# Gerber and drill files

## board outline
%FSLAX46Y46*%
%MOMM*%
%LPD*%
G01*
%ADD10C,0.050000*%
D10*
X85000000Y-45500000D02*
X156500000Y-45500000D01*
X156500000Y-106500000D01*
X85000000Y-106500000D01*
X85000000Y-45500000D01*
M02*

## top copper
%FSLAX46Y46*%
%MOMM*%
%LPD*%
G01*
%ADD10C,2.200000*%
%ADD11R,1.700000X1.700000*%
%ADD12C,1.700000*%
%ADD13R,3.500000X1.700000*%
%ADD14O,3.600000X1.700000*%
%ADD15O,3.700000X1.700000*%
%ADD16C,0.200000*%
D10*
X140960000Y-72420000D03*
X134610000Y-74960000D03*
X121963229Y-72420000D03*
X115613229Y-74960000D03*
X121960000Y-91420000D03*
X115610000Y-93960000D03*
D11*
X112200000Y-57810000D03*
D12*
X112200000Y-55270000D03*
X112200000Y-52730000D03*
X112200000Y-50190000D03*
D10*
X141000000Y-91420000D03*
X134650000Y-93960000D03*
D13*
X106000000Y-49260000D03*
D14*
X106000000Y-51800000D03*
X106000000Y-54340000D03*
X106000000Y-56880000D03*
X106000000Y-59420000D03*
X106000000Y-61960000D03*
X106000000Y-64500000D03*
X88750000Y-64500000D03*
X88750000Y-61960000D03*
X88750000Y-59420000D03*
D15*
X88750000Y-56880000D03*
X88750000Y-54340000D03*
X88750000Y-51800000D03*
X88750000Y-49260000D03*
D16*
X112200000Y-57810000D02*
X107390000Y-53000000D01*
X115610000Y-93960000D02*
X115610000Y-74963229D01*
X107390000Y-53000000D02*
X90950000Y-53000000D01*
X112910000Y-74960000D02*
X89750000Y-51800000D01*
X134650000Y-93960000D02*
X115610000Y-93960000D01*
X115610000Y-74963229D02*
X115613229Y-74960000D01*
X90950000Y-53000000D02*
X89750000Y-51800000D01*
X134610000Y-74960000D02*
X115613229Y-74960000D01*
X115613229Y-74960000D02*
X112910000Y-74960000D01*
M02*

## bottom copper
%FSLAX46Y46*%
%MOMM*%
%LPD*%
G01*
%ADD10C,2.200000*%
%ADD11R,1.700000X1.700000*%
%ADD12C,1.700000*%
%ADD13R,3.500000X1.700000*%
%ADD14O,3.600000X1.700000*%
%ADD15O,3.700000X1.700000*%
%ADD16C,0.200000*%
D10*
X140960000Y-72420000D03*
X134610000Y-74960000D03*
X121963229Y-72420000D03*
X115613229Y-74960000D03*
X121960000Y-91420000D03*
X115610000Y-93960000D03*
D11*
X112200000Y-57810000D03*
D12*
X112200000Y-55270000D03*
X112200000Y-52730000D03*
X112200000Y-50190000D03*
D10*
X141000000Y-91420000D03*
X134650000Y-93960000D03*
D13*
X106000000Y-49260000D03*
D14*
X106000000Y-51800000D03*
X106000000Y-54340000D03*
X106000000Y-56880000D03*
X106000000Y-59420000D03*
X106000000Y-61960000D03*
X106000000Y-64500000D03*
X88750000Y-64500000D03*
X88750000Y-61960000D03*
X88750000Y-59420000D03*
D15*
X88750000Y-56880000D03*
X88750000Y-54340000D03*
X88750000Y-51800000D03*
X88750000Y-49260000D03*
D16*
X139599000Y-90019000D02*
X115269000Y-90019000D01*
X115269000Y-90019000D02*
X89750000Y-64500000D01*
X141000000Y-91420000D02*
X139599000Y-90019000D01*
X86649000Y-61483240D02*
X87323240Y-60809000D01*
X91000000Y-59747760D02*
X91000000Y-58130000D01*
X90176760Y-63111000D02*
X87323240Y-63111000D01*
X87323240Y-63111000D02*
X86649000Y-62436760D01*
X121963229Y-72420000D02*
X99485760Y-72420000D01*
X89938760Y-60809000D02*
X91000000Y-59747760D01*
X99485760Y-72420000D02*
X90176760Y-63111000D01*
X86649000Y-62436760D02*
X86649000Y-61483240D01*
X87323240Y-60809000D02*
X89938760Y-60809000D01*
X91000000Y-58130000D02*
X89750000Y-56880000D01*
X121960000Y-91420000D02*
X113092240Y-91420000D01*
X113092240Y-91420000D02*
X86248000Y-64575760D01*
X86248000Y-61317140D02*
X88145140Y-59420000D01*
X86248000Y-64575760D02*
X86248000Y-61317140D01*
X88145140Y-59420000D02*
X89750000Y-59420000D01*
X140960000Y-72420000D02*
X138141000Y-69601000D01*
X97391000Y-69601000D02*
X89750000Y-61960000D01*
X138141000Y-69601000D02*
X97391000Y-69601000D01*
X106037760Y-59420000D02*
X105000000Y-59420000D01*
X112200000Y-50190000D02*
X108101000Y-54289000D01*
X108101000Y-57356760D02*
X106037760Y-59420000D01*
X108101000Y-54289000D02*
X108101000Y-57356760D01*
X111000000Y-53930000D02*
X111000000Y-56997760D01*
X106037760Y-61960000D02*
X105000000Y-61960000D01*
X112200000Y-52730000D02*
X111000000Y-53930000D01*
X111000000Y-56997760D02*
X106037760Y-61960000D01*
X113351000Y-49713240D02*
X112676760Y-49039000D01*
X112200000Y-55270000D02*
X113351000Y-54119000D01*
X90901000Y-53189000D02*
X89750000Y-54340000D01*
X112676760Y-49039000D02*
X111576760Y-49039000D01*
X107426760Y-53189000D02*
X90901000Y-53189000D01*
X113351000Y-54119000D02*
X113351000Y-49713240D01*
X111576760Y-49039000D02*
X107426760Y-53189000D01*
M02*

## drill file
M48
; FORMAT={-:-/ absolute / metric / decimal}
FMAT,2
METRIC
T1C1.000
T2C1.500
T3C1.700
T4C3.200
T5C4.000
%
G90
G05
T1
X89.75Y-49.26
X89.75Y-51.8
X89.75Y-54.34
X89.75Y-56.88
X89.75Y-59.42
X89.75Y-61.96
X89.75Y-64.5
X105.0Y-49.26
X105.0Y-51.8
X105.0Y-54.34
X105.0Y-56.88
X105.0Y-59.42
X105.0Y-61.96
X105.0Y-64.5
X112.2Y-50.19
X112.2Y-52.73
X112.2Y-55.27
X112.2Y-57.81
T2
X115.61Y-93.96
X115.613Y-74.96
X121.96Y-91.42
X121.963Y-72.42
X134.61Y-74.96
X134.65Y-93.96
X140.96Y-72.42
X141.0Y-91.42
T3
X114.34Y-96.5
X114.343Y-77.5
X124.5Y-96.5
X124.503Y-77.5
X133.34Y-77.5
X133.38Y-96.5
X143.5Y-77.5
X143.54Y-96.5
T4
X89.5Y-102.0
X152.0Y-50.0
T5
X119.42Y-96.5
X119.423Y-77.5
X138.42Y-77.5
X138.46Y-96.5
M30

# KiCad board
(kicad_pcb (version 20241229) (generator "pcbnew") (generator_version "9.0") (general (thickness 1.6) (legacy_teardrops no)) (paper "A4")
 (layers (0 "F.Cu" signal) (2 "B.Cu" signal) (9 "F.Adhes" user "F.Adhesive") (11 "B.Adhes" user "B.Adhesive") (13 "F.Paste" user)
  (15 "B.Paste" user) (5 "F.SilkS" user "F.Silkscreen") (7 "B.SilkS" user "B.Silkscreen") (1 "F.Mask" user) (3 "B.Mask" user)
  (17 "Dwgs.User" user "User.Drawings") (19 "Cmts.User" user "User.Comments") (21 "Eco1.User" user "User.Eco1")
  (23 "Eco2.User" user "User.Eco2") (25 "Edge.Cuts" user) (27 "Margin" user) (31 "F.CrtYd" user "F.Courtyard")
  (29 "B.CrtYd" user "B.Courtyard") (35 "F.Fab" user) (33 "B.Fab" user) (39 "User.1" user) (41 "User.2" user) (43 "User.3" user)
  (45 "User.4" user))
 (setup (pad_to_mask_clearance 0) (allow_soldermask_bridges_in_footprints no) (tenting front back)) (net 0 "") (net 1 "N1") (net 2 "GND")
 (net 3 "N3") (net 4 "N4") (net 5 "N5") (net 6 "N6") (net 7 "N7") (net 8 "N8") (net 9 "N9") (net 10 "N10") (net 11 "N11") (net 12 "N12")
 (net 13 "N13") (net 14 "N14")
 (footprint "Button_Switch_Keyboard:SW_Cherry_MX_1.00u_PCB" (layer "F.Cu") (at 140.96 72.42)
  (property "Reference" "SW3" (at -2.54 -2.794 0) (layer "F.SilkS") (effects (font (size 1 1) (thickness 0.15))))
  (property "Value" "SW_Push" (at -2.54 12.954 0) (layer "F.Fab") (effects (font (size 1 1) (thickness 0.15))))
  (pad "" np_thru_hole circle (at -7.62 5.08) (size 1.7 1.7) (drill 1.7) (layers "*.Cu" "*.Mask"))
  (pad "" np_thru_hole circle (at -2.54 5.08) (size 4 4) (drill 4) (layers "*.Cu" "*.Mask"))
  (pad "" np_thru_hole circle (at 2.54 5.08) (size 1.7 1.7) (drill 1.7) (layers "*.Cu" "*.Mask"))
  (pad "1" thru_hole circle (at 0 0) (size 2.2 2.2) (drill 1.5) (layers "*.Cu" "*.Mask") (remove_unused_layers no) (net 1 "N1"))
  (pad "2" thru_hole circle (at -6.35 2.54) (size 2.2 2.2) (drill 1.5) (layers "*.Cu" "*.Mask") (remove_unused_layers no) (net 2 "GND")))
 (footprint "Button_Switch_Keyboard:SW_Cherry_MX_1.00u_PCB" (layer "F.Cu") (at 121.963229 72.42)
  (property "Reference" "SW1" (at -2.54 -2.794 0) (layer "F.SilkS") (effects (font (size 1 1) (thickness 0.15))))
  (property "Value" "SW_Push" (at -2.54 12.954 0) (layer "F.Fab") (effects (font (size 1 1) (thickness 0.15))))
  (pad "" np_thru_hole circle (at -7.62 5.08) (size 1.7 1.7) (drill 1.7) (layers "*.Cu" "*.Mask"))
  (pad "" np_thru_hole circle (at -2.54 5.08) (size 4 4) (drill 4) (layers "*.Cu" "*.Mask"))
  (pad "" np_thru_hole circle (at 2.54 5.08) (size 1.7 1.7) (drill 1.7) (layers "*.Cu" "*.Mask"))
  (pad "1" thru_hole circle (at 0 0) (size 2.2 2.2) (drill 1.5) (layers "*.Cu" "*.Mask") (remove_unused_layers no) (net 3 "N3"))
  (pad "2" thru_hole circle (at -6.35 2.54) (size 2.2 2.2) (drill 1.5) (layers "*.Cu" "*.Mask") (remove_unused_layers no) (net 2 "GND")))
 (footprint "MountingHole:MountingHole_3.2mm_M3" (layer "F.Cu") (at 152 50)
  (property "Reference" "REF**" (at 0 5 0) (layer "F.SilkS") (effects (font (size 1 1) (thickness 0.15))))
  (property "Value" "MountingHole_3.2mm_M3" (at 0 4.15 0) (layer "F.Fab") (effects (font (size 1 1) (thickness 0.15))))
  (pad "" np_thru_hole circle (at 0 0) (size 3.2 3.2) (drill 3.2) (layers "*.Cu" "*.Mask")))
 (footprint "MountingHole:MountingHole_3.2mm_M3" (layer "F.Cu") (at 89.5 102)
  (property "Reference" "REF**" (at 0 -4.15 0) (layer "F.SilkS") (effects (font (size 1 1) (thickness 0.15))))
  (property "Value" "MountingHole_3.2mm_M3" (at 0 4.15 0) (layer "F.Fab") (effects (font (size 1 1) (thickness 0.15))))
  (pad "" np_thru_hole circle (at 0 0) (size 3.2 3.2) (drill 3.2) (layers "*.Cu" "*.Mask")))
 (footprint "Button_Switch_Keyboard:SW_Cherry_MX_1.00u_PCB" (layer "F.Cu") (at 121.96 91.42)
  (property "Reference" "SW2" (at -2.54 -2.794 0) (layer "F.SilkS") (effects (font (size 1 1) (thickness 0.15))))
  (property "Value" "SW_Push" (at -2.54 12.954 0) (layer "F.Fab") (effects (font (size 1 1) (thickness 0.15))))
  (pad "" np_thru_hole circle (at -7.62 5.08) (size 1.7 1.7) (drill 1.7) (layers "*.Cu" "*.Mask"))
  (pad "" np_thru_hole circle (at -2.54 5.08) (size 4 4) (drill 4) (layers "*.Cu" "*.Mask"))
  (pad "" np_thru_hole circle (at 2.54 5.08) (size 1.7 1.7) (drill 1.7) (layers "*.Cu" "*.Mask"))
  (pad "1" thru_hole circle (at 0 0) (size 2.2 2.2) (drill 1.5) (layers "*.Cu" "*.Mask") (remove_unused_layers no) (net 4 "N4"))
  (pad "2" thru_hole circle (at -6.35 2.54) (size 2.2 2.2) (drill 1.5) (layers "*.Cu" "*.Mask") (remove_unused_layers no) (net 2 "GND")))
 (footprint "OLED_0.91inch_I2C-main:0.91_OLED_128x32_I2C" (layer "F.Cu") (at 110.2 57.81)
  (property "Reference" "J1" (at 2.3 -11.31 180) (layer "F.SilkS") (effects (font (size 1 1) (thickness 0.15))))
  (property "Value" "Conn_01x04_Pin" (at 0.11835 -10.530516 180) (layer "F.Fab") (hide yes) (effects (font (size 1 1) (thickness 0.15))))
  (pad "1" thru_hole rect (at 2 0 180) (size 1.7 1.7) (drill 1) (layers "*.Cu" "*.Mask") (remove_unused_layers no) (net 2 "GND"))
  (pad "2" thru_hole circle (at 2 -2.54 180) (size 1.7 1.7) (drill 1) (layers "*.Cu" "*.Mask") (remove_unused_layers no) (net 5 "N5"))
  (pad "3" thru_hole circle (at 2 -5.08 180) (size 1.7 1.7) (drill 1) (layers "*.Cu" "*.Mask") (remove_unused_layers no) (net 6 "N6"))
  (pad "4" thru_hole circle (at 2 -7.62 180) (size 1.7 1.7) (drill 1) (layers "*.Cu" "*.Mask") (remove_unused_layers no) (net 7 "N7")))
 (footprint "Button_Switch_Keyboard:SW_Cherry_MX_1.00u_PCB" (layer "F.Cu") (at 141 91.42)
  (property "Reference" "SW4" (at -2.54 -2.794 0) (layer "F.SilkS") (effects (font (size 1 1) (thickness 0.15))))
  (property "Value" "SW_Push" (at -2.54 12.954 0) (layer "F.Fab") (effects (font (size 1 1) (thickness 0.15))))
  (pad "" np_thru_hole circle (at -7.62 5.08) (size 1.7 1.7) (drill 1.7) (layers "*.Cu" "*.Mask"))
  (pad "" np_thru_hole circle (at -2.54 5.08) (size 4 4) (drill 4) (layers "*.Cu" "*.Mask"))
  (pad "" np_thru_hole circle (at 2.54 5.08) (size 1.7 1.7) (drill 1.7) (layers "*.Cu" "*.Mask"))
  (pad "1" thru_hole circle (at 0 0) (size 2.2 2.2) (drill 1.5) (layers "*.Cu" "*.Mask") (remove_unused_layers no) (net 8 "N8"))
  (pad "2" thru_hole circle (at -6.35 2.54) (size 2.2 2.2) (drill 1.5) (layers "*.Cu" "*.Mask") (remove_unused_layers no) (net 2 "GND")))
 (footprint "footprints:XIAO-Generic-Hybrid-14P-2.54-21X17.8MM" (layer "B.Cu") (at 97.375 56.88 180)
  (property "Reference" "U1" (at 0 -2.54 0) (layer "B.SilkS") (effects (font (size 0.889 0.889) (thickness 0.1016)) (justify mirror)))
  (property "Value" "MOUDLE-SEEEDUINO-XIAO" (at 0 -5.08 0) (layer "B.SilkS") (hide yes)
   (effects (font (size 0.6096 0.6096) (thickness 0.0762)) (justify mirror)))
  (pad "1" thru_hole rect (at -7.625 7.62 180) (size 3.5 1.7) (drill 1 (offset -1 0)) (layers "*.Cu" "*.Mask") (remove_unused_layers no)
   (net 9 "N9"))
  (pad "2" thru_hole oval (at -7.625 5.08 180) (size 3.6 1.7) (drill 1 (offset -1 0)) (layers "*.Cu" "*.Mask") (remove_unused_layers no)
   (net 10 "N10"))
  (pad "3" thru_hole oval (at -7.625 2.54 180) (size 3.6 1.7) (drill 1 (offset -1 0)) (layers "*.Cu" "*.Mask") (remove_unused_layers no)
   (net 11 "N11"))
  (pad "4" thru_hole oval (at -7.625 0 180) (size 3.6 1.7) (drill 1 (offset -1 0)) (layers "*.Cu" "*.Mask") (remove_unused_layers no)
   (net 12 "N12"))
  (pad "5" thru_hole oval (at -7.625 -2.54 180) (size 3.6 1.7) (drill 1 (offset -1 0)) (layers "*.Cu" "*.Mask") (remove_unused_layers no)
   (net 7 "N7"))
  (pad "6" thru_hole oval (at -7.625 -5.08) (size 3.6 1.7) (drill 1 (offset 1 0)) (layers "*.Cu" "*.Mask") (remove_unused_layers no)
   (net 6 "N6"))
  (pad "7" thru_hole oval (at -7.625 -7.62 180) (size 3.6 1.7) (drill 1 (offset -1 0)) (layers "*.Cu" "*.Mask") (remove_unused_layers no)
   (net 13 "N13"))
  (pad "8" thru_hole oval (at 7.625 -7.62 180) (size 3.6 1.7) (drill 1 (offset 1 0)) (layers "*.Cu" "*.Mask") (remove_unused_layers no)
   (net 8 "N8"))
  (pad "9" thru_hole oval (at 7.625 -5.08 180) (size 3.6 1.7) (drill 1 (offset 1 0)) (layers "*.Cu" "*.Mask") (remove_unused_layers no)
   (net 1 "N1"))
  (pad "10" thru_hole oval (at 7.625 -2.54 180) (size 3.6 1.7) (drill 1 (offset 1 0)) (layers "*.Cu" "*.Mask") (remove_unused_layers no)
   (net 4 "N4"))
  (pad "11" thru_hole oval (at 7.625 0 180) (size 3.7 1.7) (drill 1 (offset 1 0)) (layers "*.Cu" "*.Mask") (remove_unused_layers no)
   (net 3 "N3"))
  (pad "12" thru_hole oval (at 7.625 2.54 180) (size 3.7 1.7) (drill 1 (offset 1 0)) (layers "*.Cu" "*.Mask") (remove_unused_layers no)
   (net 5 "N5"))
  (pad "13" thru_hole oval (at 7.625 5.08 180) (size 3.7 1.7) (drill 1 (offset 1 0)) (layers "*.Cu" "*.Mask") (remove_unused_layers no)
   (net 2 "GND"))
  (pad "14" thru_hole oval (at 7.625 7.62 180) (size 3.7 1.7) (drill 1 (offset 1 0)) (layers "*.Cu" "*.Mask") (remove_unused_layers no)
   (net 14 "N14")))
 (gr_rect (start 85 45.5) (end 156.5 106.5) (stroke (width 0.05) (type default)) (fill no) (layer "Edge.Cuts"))
 (segment (start 139.599 90.019) (end 115.269 90.019) (width 0.2) (layer "B.Cu") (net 8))
 (segment (start 115.269 90.019) (end 89.75 64.5) (width 0.2) (layer "B.Cu") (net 8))
 (segment (start 141 91.42) (end 139.599 90.019) (width 0.2) (layer "B.Cu") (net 8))
 (segment (start 86.649 61.48324) (end 87.32324 60.809) (width 0.2) (layer "B.Cu") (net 3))
 (segment (start 91 59.74776) (end 91 58.13) (width 0.2) (layer "B.Cu") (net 3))
 (segment (start 90.17676 63.111) (end 87.32324 63.111) (width 0.2) (layer "B.Cu") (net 3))
 (segment (start 87.32324 63.111) (end 86.649 62.43676) (width 0.2) (layer "B.Cu") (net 3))
 (segment (start 121.963229 72.42) (end 99.48576 72.42) (width 0.2) (layer "B.Cu") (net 3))
 (segment (start 89.93876 60.809) (end 91 59.74776) (width 0.2) (layer "B.Cu") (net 3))
 (segment (start 99.48576 72.42) (end 90.17676 63.111) (width 0.2) (layer "B.Cu") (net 3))
 (segment (start 86.649 62.43676) (end 86.649 61.48324) (width 0.2) (layer "B.Cu") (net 3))
 (segment (start 87.32324 60.809) (end 89.93876 60.809) (width 0.2) (layer "B.Cu") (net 3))
 (segment (start 91 58.13) (end 89.75 56.88) (width 0.2) (layer "B.Cu") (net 3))
 (segment (start 112.2 57.81) (end 107.39 53) (width 0.2) (layer "F.Cu") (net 2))
 (segment (start 115.61 93.96) (end 115.61 74.963229) (width 0.2) (layer "F.Cu") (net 2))
 (segment (start 107.39 53) (end 90.95 53) (width 0.2) (layer "F.Cu") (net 2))
 (segment (start 112.91 74.96) (end 89.75 51.8) (width 0.2) (layer "F.Cu") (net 2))
 (segment (start 134.65 93.96) (end 115.61 93.96) (width 0.2) (layer "F.Cu") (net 2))
 (segment (start 115.61 74.963229) (end 115.613229 74.96) (width 0.2) (layer "F.Cu") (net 2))
 (segment (start 90.95 53) (end 89.75 51.8) (width 0.2) (layer "F.Cu") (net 2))
 (segment (start 134.61 74.96) (end 115.613229 74.96) (width 0.2) (layer "F.Cu") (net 2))
 (segment (start 115.613229 74.96) (end 112.91 74.96) (width 0.2) (layer "F.Cu") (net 2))
 (segment (start 121.96 91.42) (end 113.09224 91.42) (width 0.2) (layer "B.Cu") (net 4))
 (segment (start 113.09224 91.42) (end 86.248 64.57576) (width 0.2) (layer "B.Cu") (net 4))
 (segment (start 86.248 61.31714) (end 88.14514 59.42) (width 0.2) (layer "B.Cu") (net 4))
 (segment (start 86.248 64.57576) (end 86.248 61.31714) (width 0.2) (layer "B.Cu") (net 4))
 (segment (start 88.14514 59.42) (end 89.75 59.42) (width 0.2) (layer "B.Cu") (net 4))
 (segment (start 140.96 72.42) (end 138.141 69.601) (width 0.2) (layer "B.Cu") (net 1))
 (segment (start 97.391 69.601) (end 89.75 61.96) (width 0.2) (layer "B.Cu") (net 1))
 (segment (start 138.141 69.601) (end 97.391 69.601) (width 0.2) (layer "B.Cu") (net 1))
 (segment (start 106.03776 59.42) (end 105 59.42) (width 0.2) (layer "B.Cu") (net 7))
 (segment (start 112.2 50.19) (end 108.101 54.289) (width 0.2) (layer "B.Cu") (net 7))
 (segment (start 108.101 57.35676) (end 106.03776 59.42) (width 0.2) (layer "B.Cu") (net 7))
 (segment (start 108.101 54.289) (end 108.101 57.35676) (width 0.2) (layer "B.Cu") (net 7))
 (segment (start 111 53.93) (end 111 56.99776) (width 0.2) (layer "B.Cu") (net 6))
 (segment (start 106.03776 61.96) (end 105 61.96) (width 0.2) (layer "B.Cu") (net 6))
 (segment (start 112.2 52.73) (end 111 53.93) (width 0.2) (layer "B.Cu") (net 6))
 (segment (start 111 56.99776) (end 106.03776 61.96) (width 0.2) (layer "B.Cu") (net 6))
 (segment (start 113.351 49.71324) (end 112.67676 49.039) (width 0.2) (layer "B.Cu") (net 5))
 (segment (start 112.2 55.27) (end 113.351 54.119) (width 0.2) (layer "B.Cu") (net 5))
 (segment (start 90.901 53.189) (end 89.75 54.34) (width 0.2) (layer "B.Cu") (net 5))
 (segment (start 112.67676 49.039) (end 111.57676 49.039) (width 0.2) (layer "B.Cu") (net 5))
 (segment (start 107.42676 53.189) (end 90.901 53.189) (width 0.2) (layer "B.Cu") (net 5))
 (segment (start 113.351 54.119) (end 113.351 49.71324) (width 0.2) (layer "B.Cu") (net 5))
 (segment (start 111.57676 49.039) (end 107.42676 53.189) (width 0.2) (layer "B.Cu") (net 5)))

